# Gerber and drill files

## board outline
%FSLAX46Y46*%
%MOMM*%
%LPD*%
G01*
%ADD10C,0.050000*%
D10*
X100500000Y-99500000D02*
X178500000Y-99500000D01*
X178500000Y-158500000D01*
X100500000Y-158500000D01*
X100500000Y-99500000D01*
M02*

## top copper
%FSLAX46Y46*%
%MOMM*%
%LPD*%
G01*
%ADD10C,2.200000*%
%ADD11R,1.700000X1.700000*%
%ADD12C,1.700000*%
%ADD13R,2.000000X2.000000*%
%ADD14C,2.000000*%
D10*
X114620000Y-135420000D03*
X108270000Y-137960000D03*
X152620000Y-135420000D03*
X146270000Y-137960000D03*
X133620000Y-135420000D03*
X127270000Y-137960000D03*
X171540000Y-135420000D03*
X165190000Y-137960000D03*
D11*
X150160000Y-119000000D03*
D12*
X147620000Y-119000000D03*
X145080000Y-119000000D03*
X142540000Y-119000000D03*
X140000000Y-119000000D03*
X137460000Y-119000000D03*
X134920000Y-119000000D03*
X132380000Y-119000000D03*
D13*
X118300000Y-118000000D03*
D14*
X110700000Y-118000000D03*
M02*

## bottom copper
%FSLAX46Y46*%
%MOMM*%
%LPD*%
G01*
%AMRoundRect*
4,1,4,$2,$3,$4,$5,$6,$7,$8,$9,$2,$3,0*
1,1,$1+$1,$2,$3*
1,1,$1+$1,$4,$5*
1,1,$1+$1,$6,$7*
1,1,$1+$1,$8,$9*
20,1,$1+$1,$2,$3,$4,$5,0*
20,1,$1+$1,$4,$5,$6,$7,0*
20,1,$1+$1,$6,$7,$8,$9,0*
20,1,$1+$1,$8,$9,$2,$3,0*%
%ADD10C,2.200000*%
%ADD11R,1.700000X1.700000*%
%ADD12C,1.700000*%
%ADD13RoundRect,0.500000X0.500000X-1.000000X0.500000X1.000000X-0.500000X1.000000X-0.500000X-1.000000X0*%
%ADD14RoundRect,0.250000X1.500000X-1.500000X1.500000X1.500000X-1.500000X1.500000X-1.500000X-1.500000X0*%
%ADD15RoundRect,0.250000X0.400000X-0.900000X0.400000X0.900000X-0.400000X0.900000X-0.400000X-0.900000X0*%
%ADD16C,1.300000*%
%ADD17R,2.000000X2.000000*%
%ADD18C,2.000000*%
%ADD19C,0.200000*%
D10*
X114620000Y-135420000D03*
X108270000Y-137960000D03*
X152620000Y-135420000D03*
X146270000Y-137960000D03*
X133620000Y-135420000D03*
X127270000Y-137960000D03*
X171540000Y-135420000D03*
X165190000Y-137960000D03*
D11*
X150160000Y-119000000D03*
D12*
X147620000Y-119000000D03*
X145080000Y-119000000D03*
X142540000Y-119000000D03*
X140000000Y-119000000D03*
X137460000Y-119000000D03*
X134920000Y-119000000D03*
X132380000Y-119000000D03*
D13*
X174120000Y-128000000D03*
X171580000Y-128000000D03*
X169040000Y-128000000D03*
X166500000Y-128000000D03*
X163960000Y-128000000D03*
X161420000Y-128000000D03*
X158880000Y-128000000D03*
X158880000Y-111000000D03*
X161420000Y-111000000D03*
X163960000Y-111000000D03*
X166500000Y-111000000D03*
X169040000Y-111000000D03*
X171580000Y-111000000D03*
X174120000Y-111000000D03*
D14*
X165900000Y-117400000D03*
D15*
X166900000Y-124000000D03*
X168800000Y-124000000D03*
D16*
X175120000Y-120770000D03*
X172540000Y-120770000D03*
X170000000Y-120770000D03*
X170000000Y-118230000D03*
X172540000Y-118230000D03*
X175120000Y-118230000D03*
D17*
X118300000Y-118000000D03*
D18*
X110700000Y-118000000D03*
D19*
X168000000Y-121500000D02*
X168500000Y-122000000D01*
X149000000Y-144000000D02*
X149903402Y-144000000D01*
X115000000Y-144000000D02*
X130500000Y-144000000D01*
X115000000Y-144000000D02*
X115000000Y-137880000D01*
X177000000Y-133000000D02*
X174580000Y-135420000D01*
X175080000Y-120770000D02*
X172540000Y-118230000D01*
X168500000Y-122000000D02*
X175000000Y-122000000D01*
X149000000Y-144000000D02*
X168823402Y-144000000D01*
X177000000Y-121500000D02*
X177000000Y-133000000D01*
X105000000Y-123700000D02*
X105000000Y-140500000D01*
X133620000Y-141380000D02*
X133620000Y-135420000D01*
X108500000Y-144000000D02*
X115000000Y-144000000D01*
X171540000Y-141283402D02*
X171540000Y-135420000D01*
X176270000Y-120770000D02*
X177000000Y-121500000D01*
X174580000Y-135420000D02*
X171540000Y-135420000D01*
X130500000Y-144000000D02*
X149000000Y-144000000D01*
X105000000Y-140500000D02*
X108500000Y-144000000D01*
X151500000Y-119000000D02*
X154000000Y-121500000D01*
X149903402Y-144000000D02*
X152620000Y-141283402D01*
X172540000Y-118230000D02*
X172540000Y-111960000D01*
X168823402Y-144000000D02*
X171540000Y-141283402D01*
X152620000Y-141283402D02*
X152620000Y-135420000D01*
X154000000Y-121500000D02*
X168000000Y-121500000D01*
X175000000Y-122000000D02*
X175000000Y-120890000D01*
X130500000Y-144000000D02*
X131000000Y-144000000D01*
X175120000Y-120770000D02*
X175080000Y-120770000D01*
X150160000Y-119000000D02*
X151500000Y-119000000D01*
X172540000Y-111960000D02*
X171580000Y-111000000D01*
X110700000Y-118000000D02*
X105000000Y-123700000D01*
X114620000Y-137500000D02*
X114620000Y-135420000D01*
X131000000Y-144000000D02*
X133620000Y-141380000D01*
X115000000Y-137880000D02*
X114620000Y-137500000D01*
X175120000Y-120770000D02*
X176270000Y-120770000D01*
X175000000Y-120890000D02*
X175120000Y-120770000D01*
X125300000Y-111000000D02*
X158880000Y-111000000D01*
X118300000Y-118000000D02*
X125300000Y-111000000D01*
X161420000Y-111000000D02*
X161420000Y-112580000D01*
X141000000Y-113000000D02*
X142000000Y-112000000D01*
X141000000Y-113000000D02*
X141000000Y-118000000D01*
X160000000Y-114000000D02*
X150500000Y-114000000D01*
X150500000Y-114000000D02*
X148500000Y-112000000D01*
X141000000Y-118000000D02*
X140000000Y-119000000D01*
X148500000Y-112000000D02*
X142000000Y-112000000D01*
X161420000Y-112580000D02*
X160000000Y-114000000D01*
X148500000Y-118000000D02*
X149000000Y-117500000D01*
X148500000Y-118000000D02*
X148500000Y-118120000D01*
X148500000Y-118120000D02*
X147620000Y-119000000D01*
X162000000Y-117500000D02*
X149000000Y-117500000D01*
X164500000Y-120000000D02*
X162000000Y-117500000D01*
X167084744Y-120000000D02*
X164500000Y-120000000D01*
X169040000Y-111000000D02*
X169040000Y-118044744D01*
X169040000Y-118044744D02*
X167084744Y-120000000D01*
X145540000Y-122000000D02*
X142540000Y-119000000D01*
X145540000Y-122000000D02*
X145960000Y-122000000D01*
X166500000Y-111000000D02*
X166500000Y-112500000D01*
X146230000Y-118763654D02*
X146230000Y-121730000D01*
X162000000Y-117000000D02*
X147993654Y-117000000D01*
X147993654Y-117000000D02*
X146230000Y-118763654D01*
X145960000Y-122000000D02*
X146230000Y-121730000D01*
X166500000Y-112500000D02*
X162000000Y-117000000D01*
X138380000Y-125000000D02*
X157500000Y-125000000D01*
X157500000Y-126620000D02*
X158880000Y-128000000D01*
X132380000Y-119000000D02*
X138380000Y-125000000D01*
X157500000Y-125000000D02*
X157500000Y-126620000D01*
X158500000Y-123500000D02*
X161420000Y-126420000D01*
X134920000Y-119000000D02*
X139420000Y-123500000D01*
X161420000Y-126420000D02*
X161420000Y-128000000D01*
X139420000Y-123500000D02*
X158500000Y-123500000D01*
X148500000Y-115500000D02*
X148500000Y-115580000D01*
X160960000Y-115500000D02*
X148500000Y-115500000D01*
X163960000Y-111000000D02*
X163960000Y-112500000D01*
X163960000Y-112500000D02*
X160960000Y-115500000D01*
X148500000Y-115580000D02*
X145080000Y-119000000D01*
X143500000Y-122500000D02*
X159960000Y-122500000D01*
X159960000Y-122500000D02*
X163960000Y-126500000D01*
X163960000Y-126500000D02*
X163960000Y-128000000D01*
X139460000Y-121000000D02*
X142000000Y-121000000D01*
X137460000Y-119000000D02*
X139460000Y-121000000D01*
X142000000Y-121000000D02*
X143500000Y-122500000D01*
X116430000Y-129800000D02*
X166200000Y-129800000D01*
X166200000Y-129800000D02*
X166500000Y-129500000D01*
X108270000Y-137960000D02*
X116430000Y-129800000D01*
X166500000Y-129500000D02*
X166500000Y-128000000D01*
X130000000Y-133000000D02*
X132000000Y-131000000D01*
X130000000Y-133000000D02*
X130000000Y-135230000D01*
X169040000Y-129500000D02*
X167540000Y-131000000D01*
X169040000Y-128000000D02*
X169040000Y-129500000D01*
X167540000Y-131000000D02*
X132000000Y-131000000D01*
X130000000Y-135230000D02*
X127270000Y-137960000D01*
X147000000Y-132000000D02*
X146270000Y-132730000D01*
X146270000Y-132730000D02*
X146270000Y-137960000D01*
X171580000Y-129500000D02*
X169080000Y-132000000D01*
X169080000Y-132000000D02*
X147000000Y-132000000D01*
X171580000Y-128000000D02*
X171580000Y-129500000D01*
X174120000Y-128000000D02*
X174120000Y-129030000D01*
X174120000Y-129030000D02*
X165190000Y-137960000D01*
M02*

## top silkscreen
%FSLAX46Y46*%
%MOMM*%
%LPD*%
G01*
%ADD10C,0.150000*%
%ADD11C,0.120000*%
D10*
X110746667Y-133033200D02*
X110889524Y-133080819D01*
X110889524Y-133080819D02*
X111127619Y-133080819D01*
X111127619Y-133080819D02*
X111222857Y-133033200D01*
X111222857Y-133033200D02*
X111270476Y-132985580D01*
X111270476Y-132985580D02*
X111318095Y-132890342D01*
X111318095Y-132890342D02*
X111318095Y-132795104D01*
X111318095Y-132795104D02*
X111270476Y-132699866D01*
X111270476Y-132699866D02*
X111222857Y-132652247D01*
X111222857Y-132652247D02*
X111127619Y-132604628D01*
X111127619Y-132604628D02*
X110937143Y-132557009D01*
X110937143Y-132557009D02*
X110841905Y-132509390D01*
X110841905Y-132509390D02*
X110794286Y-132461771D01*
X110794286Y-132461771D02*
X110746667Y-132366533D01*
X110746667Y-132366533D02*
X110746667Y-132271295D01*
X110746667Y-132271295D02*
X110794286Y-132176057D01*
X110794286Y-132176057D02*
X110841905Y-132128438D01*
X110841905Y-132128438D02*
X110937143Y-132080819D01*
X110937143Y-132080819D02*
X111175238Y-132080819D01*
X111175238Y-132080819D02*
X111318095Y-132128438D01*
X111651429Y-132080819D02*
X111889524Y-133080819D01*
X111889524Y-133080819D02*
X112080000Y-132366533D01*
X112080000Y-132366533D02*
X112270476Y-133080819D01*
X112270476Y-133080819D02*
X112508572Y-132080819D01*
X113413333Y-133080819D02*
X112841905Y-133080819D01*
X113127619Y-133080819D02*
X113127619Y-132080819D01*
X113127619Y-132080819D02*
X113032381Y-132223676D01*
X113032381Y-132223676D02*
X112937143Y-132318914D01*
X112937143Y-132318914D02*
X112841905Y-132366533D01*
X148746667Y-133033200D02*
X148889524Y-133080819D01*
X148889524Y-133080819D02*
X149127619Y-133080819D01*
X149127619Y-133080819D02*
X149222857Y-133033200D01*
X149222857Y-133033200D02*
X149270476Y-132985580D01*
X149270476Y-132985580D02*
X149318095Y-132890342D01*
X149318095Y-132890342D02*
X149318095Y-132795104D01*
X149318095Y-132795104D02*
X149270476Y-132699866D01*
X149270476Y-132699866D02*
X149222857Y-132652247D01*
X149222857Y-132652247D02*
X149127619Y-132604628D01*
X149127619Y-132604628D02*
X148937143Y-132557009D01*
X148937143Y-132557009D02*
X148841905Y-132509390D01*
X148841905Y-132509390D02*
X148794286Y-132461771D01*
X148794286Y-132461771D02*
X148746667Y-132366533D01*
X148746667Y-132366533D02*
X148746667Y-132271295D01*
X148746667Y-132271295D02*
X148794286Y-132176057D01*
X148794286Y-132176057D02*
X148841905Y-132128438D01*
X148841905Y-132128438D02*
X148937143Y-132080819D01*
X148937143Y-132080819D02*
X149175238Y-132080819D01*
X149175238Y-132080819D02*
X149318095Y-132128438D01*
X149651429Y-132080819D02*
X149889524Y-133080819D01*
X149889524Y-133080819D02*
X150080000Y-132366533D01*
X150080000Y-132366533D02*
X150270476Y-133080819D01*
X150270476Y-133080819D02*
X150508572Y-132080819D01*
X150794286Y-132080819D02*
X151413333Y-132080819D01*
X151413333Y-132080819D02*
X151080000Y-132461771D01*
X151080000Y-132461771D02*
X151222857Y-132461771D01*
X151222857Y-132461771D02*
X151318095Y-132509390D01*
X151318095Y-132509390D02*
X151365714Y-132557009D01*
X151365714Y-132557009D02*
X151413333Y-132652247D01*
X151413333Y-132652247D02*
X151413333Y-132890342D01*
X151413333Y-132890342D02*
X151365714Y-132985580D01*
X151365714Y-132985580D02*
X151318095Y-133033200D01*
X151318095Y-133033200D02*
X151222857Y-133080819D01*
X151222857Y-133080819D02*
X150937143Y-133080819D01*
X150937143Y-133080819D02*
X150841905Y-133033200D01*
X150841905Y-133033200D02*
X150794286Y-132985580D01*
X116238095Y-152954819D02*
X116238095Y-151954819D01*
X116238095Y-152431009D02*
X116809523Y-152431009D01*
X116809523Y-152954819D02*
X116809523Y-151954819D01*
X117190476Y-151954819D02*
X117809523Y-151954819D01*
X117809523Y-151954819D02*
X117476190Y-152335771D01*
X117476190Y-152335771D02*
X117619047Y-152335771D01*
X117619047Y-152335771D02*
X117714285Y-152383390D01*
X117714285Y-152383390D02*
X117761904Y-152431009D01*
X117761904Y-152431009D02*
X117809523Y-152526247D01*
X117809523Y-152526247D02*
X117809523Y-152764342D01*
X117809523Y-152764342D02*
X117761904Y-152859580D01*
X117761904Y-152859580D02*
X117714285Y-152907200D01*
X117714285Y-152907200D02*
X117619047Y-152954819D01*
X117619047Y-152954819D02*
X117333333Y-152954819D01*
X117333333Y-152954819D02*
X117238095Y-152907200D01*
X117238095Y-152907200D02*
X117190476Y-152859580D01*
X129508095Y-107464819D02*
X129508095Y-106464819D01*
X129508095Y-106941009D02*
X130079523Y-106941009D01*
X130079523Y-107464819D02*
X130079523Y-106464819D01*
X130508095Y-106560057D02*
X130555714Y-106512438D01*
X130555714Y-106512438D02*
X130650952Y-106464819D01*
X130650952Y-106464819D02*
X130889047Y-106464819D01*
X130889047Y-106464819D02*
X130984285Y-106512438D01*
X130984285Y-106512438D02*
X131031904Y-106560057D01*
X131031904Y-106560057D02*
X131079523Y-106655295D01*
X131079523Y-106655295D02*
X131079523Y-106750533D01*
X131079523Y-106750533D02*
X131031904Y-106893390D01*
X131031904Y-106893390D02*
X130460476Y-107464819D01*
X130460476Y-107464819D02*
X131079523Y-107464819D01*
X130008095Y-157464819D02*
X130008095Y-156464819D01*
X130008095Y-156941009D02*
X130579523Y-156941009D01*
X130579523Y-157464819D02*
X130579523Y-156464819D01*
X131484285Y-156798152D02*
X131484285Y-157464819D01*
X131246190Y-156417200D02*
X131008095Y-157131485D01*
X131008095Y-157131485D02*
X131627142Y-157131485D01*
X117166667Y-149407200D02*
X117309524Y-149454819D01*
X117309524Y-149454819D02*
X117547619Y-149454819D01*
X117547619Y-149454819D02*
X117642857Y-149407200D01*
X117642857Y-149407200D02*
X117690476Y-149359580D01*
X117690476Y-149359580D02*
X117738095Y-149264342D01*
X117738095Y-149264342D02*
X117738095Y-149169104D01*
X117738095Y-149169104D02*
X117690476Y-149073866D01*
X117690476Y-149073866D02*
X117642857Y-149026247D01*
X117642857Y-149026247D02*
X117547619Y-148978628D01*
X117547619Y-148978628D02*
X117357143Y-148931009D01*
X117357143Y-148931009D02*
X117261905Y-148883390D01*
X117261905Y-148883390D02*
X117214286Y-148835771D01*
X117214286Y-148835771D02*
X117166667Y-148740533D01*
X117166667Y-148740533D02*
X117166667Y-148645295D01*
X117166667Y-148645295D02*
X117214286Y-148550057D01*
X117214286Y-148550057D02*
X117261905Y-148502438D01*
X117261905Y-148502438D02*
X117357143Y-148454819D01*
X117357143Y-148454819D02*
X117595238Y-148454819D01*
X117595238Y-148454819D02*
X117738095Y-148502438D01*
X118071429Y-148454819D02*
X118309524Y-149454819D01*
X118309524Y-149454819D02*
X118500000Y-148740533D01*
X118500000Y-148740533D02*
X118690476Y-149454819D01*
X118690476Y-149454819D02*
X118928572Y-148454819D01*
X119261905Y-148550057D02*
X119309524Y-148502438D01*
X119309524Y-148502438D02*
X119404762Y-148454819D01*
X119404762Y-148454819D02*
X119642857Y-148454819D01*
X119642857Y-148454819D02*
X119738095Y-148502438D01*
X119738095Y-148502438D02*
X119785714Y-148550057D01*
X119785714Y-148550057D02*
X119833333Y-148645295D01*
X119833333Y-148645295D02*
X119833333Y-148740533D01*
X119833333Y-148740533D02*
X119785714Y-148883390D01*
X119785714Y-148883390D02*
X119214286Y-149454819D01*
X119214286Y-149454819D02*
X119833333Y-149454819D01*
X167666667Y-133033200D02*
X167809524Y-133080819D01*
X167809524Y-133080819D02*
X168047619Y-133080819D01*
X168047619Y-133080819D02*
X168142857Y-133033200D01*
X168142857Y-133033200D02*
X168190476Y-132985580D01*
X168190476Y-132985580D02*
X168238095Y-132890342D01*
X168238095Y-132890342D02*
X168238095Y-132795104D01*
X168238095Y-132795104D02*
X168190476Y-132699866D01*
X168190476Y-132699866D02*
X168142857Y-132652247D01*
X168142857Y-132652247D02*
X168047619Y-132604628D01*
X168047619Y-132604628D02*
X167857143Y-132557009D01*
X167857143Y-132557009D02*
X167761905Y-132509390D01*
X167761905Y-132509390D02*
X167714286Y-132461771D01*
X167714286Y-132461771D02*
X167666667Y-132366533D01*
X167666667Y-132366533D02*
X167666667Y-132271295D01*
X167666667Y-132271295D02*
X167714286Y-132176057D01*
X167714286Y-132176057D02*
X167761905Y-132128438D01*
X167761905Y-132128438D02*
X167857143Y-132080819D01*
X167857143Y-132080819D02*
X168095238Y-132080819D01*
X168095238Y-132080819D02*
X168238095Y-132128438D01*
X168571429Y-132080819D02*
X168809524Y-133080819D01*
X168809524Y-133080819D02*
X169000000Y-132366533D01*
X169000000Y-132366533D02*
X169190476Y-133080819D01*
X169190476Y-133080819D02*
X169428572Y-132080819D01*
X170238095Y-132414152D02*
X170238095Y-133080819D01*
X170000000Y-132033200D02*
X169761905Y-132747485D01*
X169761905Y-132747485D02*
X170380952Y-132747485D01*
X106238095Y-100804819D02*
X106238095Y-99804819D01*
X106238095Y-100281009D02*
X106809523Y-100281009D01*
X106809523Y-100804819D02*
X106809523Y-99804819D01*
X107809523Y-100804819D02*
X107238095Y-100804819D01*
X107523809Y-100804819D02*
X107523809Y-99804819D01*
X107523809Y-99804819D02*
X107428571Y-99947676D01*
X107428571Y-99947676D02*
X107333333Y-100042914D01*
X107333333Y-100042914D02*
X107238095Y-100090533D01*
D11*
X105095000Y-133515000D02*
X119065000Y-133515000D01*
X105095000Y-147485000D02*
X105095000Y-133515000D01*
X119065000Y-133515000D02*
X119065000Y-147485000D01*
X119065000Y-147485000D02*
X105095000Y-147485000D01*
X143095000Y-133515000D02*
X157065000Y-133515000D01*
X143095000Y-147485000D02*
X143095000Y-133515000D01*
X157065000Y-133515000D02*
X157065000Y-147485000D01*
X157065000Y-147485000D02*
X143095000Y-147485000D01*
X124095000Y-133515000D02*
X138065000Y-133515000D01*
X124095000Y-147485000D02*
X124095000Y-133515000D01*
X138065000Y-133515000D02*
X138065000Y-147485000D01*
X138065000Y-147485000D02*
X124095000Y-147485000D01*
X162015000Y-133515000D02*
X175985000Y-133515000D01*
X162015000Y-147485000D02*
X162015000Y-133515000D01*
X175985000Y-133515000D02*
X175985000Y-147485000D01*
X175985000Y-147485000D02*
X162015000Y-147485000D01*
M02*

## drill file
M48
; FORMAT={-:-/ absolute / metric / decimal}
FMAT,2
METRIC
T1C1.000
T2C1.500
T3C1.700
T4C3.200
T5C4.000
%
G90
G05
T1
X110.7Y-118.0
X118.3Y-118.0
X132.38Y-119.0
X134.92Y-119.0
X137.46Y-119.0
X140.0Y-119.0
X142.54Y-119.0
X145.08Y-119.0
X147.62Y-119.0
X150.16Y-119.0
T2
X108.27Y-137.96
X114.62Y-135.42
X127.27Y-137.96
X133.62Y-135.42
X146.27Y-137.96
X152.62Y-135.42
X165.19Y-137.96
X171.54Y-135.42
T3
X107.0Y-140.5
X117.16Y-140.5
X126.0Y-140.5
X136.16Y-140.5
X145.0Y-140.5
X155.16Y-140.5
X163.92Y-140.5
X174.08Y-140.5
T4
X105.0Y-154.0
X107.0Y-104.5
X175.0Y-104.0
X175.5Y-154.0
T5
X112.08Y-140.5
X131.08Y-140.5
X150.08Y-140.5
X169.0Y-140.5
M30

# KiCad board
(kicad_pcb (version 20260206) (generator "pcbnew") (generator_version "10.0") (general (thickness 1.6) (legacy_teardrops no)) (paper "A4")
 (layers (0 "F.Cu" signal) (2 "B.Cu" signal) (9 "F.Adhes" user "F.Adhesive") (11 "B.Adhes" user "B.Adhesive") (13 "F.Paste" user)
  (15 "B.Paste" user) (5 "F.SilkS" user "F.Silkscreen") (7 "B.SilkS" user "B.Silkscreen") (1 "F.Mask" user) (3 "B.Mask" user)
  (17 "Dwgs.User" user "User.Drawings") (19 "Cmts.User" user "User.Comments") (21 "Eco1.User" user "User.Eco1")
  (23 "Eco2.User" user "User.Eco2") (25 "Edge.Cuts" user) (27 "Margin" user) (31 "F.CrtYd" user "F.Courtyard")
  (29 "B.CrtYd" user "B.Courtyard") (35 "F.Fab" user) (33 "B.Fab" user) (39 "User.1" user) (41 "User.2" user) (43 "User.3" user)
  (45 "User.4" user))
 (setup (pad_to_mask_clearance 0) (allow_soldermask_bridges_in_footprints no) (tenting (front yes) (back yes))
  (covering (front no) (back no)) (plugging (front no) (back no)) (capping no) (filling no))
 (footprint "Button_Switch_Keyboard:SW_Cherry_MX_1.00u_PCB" (layer "F.Cu") (at 114.62 135.42)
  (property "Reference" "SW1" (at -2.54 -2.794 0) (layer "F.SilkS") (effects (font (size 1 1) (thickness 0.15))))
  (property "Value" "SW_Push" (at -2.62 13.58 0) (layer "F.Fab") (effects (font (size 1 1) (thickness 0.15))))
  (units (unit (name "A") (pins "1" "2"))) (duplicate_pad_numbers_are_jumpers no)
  (fp_line (start -9.525 -1.905) (end 4.445 -1.905) (stroke (width 0.12) (type solid)) (layer "F.SilkS"))
  (fp_line (start -9.525 12.065) (end -9.525 -1.905) (stroke (width 0.12) (type solid)) (layer "F.SilkS"))
  (fp_line (start 4.445 -1.905) (end 4.445 12.065) (stroke (width 0.12) (type solid)) (layer "F.SilkS"))
  (fp_line (start 4.445 12.065) (end -9.525 12.065) (stroke (width 0.12) (type solid)) (layer "F.SilkS"))
  (pad "" np_thru_hole circle (at -7.62 5.08) (size 1.7 1.7) (drill 1.7) (layers "*.Cu" "*.Mask"))
  (pad "" np_thru_hole circle (at -2.54 5.08) (size 4 4) (drill 4) (layers "*.Cu" "*.Mask"))
  (pad "" np_thru_hole circle (at 2.54 5.08) (size 1.7 1.7) (drill 1.7) (layers "*.Cu" "*.Mask"))
  (pad "1" thru_hole circle (at 0 0) (size 2.2 2.2) (drill 1.5) (layers "*.Cu" "*.Mask") (remove_unused_layers no) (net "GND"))
  (pad "2" thru_hole circle (at -6.35 2.54) (size 2.2 2.2) (drill 1.5) (layers "*.Cu" "*.Mask") (remove_unused_layers no)
   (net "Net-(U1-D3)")))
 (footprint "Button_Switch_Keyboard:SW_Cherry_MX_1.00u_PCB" (layer "F.Cu") (at 152.62 135.42)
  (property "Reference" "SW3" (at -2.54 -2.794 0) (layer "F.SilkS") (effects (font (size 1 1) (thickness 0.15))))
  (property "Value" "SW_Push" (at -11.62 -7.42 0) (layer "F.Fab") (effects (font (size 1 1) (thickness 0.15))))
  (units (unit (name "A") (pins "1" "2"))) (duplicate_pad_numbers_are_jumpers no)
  (fp_line (start -9.525 -1.905) (end 4.445 -1.905) (stroke (width 0.12) (type solid)) (layer "F.SilkS"))
  (fp_line (start -9.525 12.065) (end -9.525 -1.905) (stroke (width 0.12) (type solid)) (layer "F.SilkS"))
  (fp_line (start 4.445 -1.905) (end 4.445 12.065) (stroke (width 0.12) (type solid)) (layer "F.SilkS"))
  (fp_line (start 4.445 12.065) (end -9.525 12.065) (stroke (width 0.12) (type solid)) (layer "F.SilkS"))
  (pad "" np_thru_hole circle (at -7.62 5.08) (size 1.7 1.7) (drill 1.7) (layers "*.Cu" "*.Mask"))
  (pad "" np_thru_hole circle (at -2.54 5.08) (size 4 4) (drill 4) (layers "*.Cu" "*.Mask"))
  (pad "" np_thru_hole circle (at 2.54 5.08) (size 1.7 1.7) (drill 1.7) (layers "*.Cu" "*.Mask"))
  (pad "1" thru_hole circle (at 0 0) (size 2.2 2.2) (drill 1.5) (layers "*.Cu" "*.Mask") (remove_unused_layers no) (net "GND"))
  (pad "2" thru_hole circle (at -6.35 2.54) (size 2.2 2.2) (drill 1.5) (layers "*.Cu" "*.Mask") (remove_unused_layers no)
   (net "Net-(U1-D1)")))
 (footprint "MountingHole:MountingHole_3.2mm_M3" (layer "F.Cu") (at 105 154)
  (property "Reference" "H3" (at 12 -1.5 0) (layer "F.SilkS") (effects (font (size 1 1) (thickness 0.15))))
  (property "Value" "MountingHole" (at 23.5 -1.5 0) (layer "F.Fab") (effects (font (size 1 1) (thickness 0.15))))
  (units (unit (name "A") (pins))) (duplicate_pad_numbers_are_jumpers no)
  (pad "" np_thru_hole circle (at 0 0) (size 3.2 3.2) (drill 3.2) (layers "*.Cu" "*.Mask")))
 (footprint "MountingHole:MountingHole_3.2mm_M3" (layer "F.Cu") (at 175 104)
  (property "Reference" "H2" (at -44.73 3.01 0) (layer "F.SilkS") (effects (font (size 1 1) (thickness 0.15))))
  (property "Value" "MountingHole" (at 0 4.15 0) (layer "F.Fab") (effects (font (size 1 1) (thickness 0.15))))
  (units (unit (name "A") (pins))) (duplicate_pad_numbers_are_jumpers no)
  (pad "" np_thru_hole circle (at 0 0) (size 3.2 3.2) (drill 3.2) (layers "*.Cu" "*.Mask")))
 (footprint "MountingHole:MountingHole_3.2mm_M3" (layer "F.Cu") (at 175.5 154)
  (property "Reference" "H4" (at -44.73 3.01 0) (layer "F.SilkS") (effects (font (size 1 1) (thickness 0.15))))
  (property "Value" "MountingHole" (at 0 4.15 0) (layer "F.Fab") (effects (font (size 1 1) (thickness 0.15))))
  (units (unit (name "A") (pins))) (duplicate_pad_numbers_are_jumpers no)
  (pad "" np_thru_hole circle (at 0 0) (size 3.2 3.2) (drill 3.2) (layers "*.Cu" "*.Mask")))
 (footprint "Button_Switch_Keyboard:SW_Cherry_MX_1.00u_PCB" (layer "F.Cu") (at 133.62 135.42)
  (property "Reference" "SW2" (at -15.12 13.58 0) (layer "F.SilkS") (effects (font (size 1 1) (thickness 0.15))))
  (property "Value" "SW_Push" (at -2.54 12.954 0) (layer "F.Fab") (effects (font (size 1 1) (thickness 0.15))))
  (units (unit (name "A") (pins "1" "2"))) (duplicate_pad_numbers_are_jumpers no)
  (fp_line (start -9.525 -1.905) (end 4.445 -1.905) (stroke (width 0.12) (type solid)) (layer "F.SilkS"))
  (fp_line (start -9.525 12.065) (end -9.525 -1.905) (stroke (width 0.12) (type solid)) (layer "F.SilkS"))
  (fp_line (start 4.445 -1.905) (end 4.445 12.065) (stroke (width 0.12) (type solid)) (layer "F.SilkS"))
  (fp_line (start 4.445 12.065) (end -9.525 12.065) (stroke (width 0.12) (type solid)) (layer "F.SilkS"))
  (pad "" np_thru_hole circle (at -7.62 5.08) (size 1.7 1.7) (drill 1.7) (layers "*.Cu" "*.Mask"))
  (pad "" np_thru_hole circle (at -2.54 5.08) (size 4 4) (drill 4) (layers "*.Cu" "*.Mask"))
  (pad "" np_thru_hole circle (at 2.54 5.08) (size 1.7 1.7) (drill 1.7) (layers "*.Cu" "*.Mask"))
  (pad "1" thru_hole circle (at 0 0) (size 2.2 2.2) (drill 1.5) (layers "*.Cu" "*.Mask") (remove_unused_layers no) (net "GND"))
  (pad "2" thru_hole circle (at -6.35 2.54) (size 2.2 2.2) (drill 1.5) (layers "*.Cu" "*.Mask") (remove_unused_layers no)
   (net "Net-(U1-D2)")))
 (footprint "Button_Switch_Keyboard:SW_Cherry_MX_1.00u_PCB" (layer "F.Cu") (at 171.54 135.42)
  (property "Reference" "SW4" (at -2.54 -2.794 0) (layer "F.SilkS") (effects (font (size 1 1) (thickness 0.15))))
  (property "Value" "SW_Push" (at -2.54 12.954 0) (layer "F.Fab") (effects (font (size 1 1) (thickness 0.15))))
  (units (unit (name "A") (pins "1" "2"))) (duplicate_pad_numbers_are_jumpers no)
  (fp_line (start -9.525 -1.905) (end 4.445 -1.905) (stroke (width 0.12) (type solid)) (layer "F.SilkS"))
  (fp_line (start -9.525 12.065) (end -9.525 -1.905) (stroke (width 0.12) (type solid)) (layer "F.SilkS"))
  (fp_line (start 4.445 -1.905) (end 4.445 12.065) (stroke (width 0.12) (type solid)) (layer "F.SilkS"))
  (fp_line (start 4.445 12.065) (end -9.525 12.065) (stroke (width 0.12) (type solid)) (layer "F.SilkS"))
  (pad "" np_thru_hole circle (at -7.62 5.08) (size 1.7 1.7) (drill 1.7) (layers "*.Cu" "*.Mask"))
  (pad "" np_thru_hole circle (at -2.54 5.08) (size 4 4) (drill 4) (layers "*.Cu" "*.Mask"))
  (pad "" np_thru_hole circle (at 2.54 5.08) (size 1.7 1.7) (drill 1.7) (layers "*.Cu" "*.Mask"))
  (pad "1" thru_hole circle (at 0 0) (size 2.2 2.2) (drill 1.5) (layers "*.Cu" "*.Mask") (remove_unused_layers no) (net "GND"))
  (pad "2" thru_hole circle (at -6.35 2.54) (size 2.2 2.2) (drill 1.5) (layers "*.Cu" "*.Mask") (remove_unused_layers no)
   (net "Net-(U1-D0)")))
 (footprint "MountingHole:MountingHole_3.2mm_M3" (layer "F.Cu") (at 107 104.5)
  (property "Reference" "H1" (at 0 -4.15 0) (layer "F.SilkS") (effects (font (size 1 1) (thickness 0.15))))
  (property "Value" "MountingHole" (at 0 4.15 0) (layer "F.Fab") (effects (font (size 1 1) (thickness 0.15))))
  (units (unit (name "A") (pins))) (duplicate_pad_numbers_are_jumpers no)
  (pad "" np_thru_hole circle (at 0 0) (size 3.2 3.2) (drill 3.2) (layers "*.Cu" "*.Mask")))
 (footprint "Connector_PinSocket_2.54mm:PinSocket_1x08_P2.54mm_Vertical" (layer "B.Cu") (at 150.16 119 90)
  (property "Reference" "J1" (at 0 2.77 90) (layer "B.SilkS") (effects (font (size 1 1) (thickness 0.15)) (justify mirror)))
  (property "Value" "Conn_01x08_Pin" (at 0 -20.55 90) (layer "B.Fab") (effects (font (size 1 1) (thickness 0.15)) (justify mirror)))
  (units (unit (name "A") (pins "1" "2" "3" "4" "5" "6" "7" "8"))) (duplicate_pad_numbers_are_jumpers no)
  (pad "1" thru_hole rect (at 0 0 90) (size 1.7 1.7) (drill 1) (layers "*.Cu" "*.Mask") (remove_unused_layers no) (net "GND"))
  (pad "2" thru_hole circle (at 0 -2.54 90) (size 1.7 1.7) (drill 1) (layers "*.Cu" "*.Mask") (remove_unused_layers no) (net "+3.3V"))
  (pad "3" thru_hole circle (at 0 -5.08 90) (size 1.7 1.7) (drill 1) (layers "*.Cu" "*.Mask") (remove_unused_layers no) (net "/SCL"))
  (pad "4" thru_hole circle (at 0 -7.62 90) (size 1.7 1.7) (drill 1) (layers "*.Cu" "*.Mask") (remove_unused_layers no) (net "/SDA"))
  (pad "5" thru_hole circle (at 0 -10.16 90) (size 1.7 1.7) (drill 1) (layers "*.Cu" "*.Mask") (remove_unused_layers no) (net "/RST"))
  (pad "6" thru_hole circle (at 0 -12.7 90) (size 1.7 1.7) (drill 1) (layers "*.Cu" "*.Mask") (remove_unused_layers no) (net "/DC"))
  (pad "7" thru_hole circle (at 0 -15.24 90) (size 1.7 1.7) (drill 1) (layers "*.Cu" "*.Mask") (remove_unused_layers no) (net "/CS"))
  (pad "8" thru_hole circle (at 0 -17.78 90) (size 1.7 1.7) (drill 1) (layers "*.Cu" "*.Mask") (remove_unused_layers no) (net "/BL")))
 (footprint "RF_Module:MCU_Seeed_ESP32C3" (layer "B.Cu") (at 166.5 119.5 90)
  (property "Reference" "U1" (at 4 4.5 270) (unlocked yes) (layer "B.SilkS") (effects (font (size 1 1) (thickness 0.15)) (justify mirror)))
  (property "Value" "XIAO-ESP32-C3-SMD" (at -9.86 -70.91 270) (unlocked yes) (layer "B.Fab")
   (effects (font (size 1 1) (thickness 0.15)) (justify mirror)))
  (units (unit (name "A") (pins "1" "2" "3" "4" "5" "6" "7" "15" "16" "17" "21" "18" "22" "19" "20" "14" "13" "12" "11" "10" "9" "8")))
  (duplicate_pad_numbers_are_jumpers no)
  (pad "" smd roundrect (at 1.1 -1.6 90) (size 1.5 1.5) (layers "B.Paste") (roundrect_rratio 0.1666666667))
  (pad "" smd roundrect (at 1.1 0.4 90) (size 1.5 1.5) (layers "B.Paste") (roundrect_rratio 0.1666666667))
  (pad "" smd roundrect (at 3.1 -1.6 90) (size 1.5 1.5) (layers "B.Paste") (roundrect_rratio 0.1666666667))
  (pad "" smd roundrect (at 3.1 0.4 90) (size 1.5 1.5) (layers "B.Paste") (roundrect_rratio 0.1666666667))
  (pad "1" smd roundrect (at -8.5 7.62 90) (size 3 2) (layers "B.Cu" "B.Mask" "B.Paste") (roundrect_rratio 0.25) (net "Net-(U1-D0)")
   (thermal_bridge_angle 45))
  (pad "2" smd roundrect (at -8.5 5.08 90) (size 3 2) (layers "B.Cu" "B.Mask" "B.Paste") (roundrect_rratio 0.25) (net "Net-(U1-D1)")
   (thermal_bridge_angle 45))
  (pad "3" smd roundrect (at -8.5 2.54 90) (size 3 2) (layers "B.Cu" "B.Mask" "B.Paste") (roundrect_rratio 0.25) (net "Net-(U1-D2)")
   (thermal_bridge_angle 45))
  (pad "4" smd roundrect (at -8.5 0 90) (size 3 2) (layers "B.Cu" "B.Mask" "B.Paste") (roundrect_rratio 0.25) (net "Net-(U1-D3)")
   (thermal_bridge_angle 45))
  (pad "5" smd roundrect (at -8.5 -2.54 90) (size 3 2) (layers "B.Cu" "B.Mask" "B.Paste") (roundrect_rratio 0.25) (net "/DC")
   (thermal_bridge_angle 45))
  (pad "6" smd roundrect (at -8.5 -5.08 90) (size 3 2) (layers "B.Cu" "B.Mask" "B.Paste") (roundrect_rratio 0.25) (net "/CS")
   (thermal_bridge_angle 45))
  (pad "7" smd roundrect (at -8.5 -7.62 90) (size 3 2) (layers "B.Cu" "B.Mask" "B.Paste") (roundrect_rratio 0.25) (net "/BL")
   (thermal_bridge_angle 45))
  (pad "8" smd roundrect (at 8.5 -7.62 90) (size 3 2) (layers "B.Cu" "B.Mask" "B.Paste") (roundrect_rratio 0.25) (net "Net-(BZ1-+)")
   (thermal_bridge_angle 45))
  (pad "9" smd roundrect (at 8.5 -5.08 90) (size 3 2) (layers "B.Cu" "B.Mask" "B.Paste") (roundrect_rratio 0.25) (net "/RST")
   (thermal_bridge_angle 45))
  (pad "10" smd roundrect (at 8.5 -2.54 90) (size 3 2) (layers "B.Cu" "B.Mask" "B.Paste") (roundrect_rratio 0.25) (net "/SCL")
   (thermal_bridge_angle 45))
  (pad "11" smd roundrect (at 8.5 0 90) (size 3 2) (layers "B.Cu" "B.Mask" "B.Paste") (roundrect_rratio 0.25) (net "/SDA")
   (thermal_bridge_angle 45))
  (pad "12" smd roundrect (at 8.5 2.54 90) (size 3 2) (layers "B.Cu" "B.Mask" "B.Paste") (roundrect_rratio 0.25) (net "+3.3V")
   (thermal_bridge_angle 45))
  (pad "13" smd roundrect (at 8.5 5.08 90) (size 3 2) (layers "B.Cu" "B.Mask" "B.Paste") (roundrect_rratio 0.25) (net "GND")
   (thermal_bridge_angle 45))
  (pad "14" smd roundrect (at 8.5 7.62 90) (size 3 2) (layers "B.Cu" "B.Mask" "B.Paste") (roundrect_rratio 0.25)
   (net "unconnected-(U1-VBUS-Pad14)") (thermal_bridge_angle 45))
  (pad "15" smd roundrect (at 2.1 -0.6 90) (size 3.5 3.5) (layers "B.Cu" "B.Mask") (roundrect_rratio 0.07142857143)
   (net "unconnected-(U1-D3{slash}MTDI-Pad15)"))
  (pad "16" smd roundrect (at -4.5 0.4 90) (size 2.3 1.3) (layers "B.Cu" "B.Mask" "B.Paste") (roundrect_rratio 0.1923076923)
   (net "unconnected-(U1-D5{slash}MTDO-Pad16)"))
  (pad "17" smd roundrect (at -4.5 2.3 90) (size 2.3 1.3) (layers "B.Cu" "B.Mask" "B.Paste") (roundrect_rratio 0.1923076923)
   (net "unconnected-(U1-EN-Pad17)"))
  (pad "18" smd circle (at -1.27 8.62 90) (size 1.3 1.3) (layers "B.Cu" "B.Mask" "B.Paste") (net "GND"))
  (pad "19" smd circle (at -1.27 6.04 90) (size 1.3 1.3) (layers "B.Cu" "B.Mask" "B.Paste") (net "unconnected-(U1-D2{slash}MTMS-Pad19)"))
  (pad "20" smd circle (at -1.27 3.5 90) (size 1.3 1.3) (layers "B.Cu" "B.Mask" "B.Paste") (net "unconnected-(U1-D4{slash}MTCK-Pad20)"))
  (pad "21" smd circle (at 1.27 3.5 90) (size 1.3 1.3) (layers "B.Cu" "B.Mask" "B.Paste") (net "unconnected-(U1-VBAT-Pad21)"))
  (pad "22" smd circle (at 1.27 6.04 90) (size 1.3 1.3) (layers "B.Cu" "B.Mask" "B.Paste") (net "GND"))
  (pad "23" smd circle (at 1.27 8.62 90) (size 1.3 1.3) (layers "B.Cu" "B.Mask" "B.Paste")))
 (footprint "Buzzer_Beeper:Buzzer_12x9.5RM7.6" (layer "B.Cu") (at 118.3 118 180)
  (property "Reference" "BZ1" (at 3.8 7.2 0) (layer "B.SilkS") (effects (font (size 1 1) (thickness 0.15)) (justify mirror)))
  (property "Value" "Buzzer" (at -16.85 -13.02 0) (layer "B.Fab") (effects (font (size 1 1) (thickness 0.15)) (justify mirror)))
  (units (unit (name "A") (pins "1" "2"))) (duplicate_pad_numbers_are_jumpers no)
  (pad "1" thru_hole rect (at 0 0 180) (size 2 2) (drill 1) (layers "*.Cu" "*.Mask") (remove_unused_layers no) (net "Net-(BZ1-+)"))
  (pad "2" thru_hole circle (at 7.6 0 180) (size 2 2) (drill 1) (layers "*.Cu" "*.Mask") (remove_unused_layers no) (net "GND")))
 (gr_rect (start 100.5 99.5) (end 178.5 158.5) (stroke (width 0.05) (type default)) (fill no) (layer "Edge.Cuts"))
 (segment (start 168 121.5) (end 168.5 122) (width 0.2) (layer "B.Cu") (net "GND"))
 (segment (start 149 144) (end 149.903402 144) (width 0.2) (layer "B.Cu") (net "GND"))
 (segment (start 115 144) (end 130.5 144) (width 0.2) (layer "B.Cu") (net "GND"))
 (segment (start 115 144) (end 115 137.88) (width 0.2) (layer "B.Cu") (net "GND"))
 (segment (start 177 133) (end 174.58 135.42) (width 0.2) (layer "B.Cu") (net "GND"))
 (segment (start 175.08 120.77) (end 172.54 118.23) (width 0.2) (layer "B.Cu") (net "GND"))
 (segment (start 168.5 122) (end 175 122) (width 0.2) (layer "B.Cu") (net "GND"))
 (segment (start 149 144) (end 168.823402 144) (width 0.2) (layer "B.Cu") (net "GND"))
 (segment (start 177 121.5) (end 177 133) (width 0.2) (layer "B.Cu") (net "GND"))
 (segment (start 105 123.7) (end 105 140.5) (width 0.2) (layer "B.Cu") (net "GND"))
 (segment (start 133.62 141.38) (end 133.62 135.42) (width 0.2) (layer "B.Cu") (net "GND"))
 (segment (start 108.5 144) (end 115 144) (width 0.2) (layer "B.Cu") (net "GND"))
 (segment (start 171.54 141.283402) (end 171.54 135.42) (width 0.2) (layer "B.Cu") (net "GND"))
 (segment (start 176.27 120.77) (end 177 121.5) (width 0.2) (layer "B.Cu") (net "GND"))
 (segment (start 174.58 135.42) (end 171.54 135.42) (width 0.2) (layer "B.Cu") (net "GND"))
 (segment (start 130.5 144) (end 149 144) (width 0.2) (layer "B.Cu") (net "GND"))
 (segment (start 105 140.5) (end 108.5 144) (width 0.2) (layer "B.Cu") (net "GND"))
 (segment (start 151.5 119) (end 154 121.5) (width 0.2) (layer "B.Cu") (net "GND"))
 (segment (start 149.903402 144) (end 152.62 141.283402) (width 0.2) (layer "B.Cu") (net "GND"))
 (segment (start 172.54 118.23) (end 172.54 111.96) (width 0.2) (layer "B.Cu") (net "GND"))
 (segment (start 168.823402 144) (end 171.54 141.283402) (width 0.2) (layer "B.Cu") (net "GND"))
 (segment (start 152.62 141.283402) (end 152.62 135.42) (width 0.2) (layer "B.Cu") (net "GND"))
 (segment (start 154 121.5) (end 168 121.5) (width 0.2) (layer "B.Cu") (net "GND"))
 (segment (start 175 122) (end 175 120.89) (width 0.2) (layer "B.Cu") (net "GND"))
 (segment (start 130.5 144) (end 131 144) (width 0.2) (layer "B.Cu") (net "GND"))
 (segment (start 175.12 120.77) (end 175.08 120.77) (width 0.2) (layer "B.Cu") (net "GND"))
 (segment (start 150.16 119) (end 151.5 119) (width 0.2) (layer "B.Cu") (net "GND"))
 (segment (start 172.54 111.96) (end 171.58 111) (width 0.2) (layer "B.Cu") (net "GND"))
 (segment (start 110.7 118) (end 105 123.7) (width 0.2) (layer "B.Cu") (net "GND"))
 (segment (start 114.62 137.5) (end 114.62 135.42) (width 0.2) (layer "B.Cu") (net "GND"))
 (segment (start 131 144) (end 133.62 141.38) (width 0.2) (layer "B.Cu") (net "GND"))
 (segment (start 115 137.88) (end 114.62 137.5) (width 0.2) (layer "B.Cu") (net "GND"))
 (segment (start 175.12 120.77) (end 176.27 120.77) (width 0.2) (layer "B.Cu") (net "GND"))
 (segment (start 175 120.89) (end 175.12 120.77) (width 0.2) (layer "B.Cu") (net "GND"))
 (segment (start 125.3 111) (end 158.88 111) (width 0.2) (layer "B.Cu") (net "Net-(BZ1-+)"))
 (segment (start 118.3 118) (end 125.3 111) (width 0.2) (layer "B.Cu") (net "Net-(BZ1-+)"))
 (segment (start 161.42 111) (end 161.42 112.58) (width 0.2) (layer "B.Cu") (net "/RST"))
 (segment (start 141 113) (end 142 112) (width 0.2) (layer "B.Cu") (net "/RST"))
 (segment (start 141 113) (end 141 118) (width 0.2) (layer "B.Cu") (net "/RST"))
 (segment (start 160 114) (end 150.5 114) (width 0.2) (layer "B.Cu") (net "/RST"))
 (segment (start 150.5 114) (end 148.5 112) (width 0.2) (layer "B.Cu") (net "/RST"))
 (segment (start 141 118) (end 140 119) (width 0.2) (layer "B.Cu") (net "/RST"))
 (segment (start 148.5 112) (end 142 112) (width 0.2) (layer "B.Cu") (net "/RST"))
 (segment (start 161.42 112.58) (end 160 114) (width 0.2) (layer "B.Cu") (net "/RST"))
 (segment (start 148.5 118) (end 149 117.5) (width 0.2) (layer "B.Cu") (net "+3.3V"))
 (segment (start 148.5 118) (end 148.5 118.12) (width 0.2) (layer "B.Cu") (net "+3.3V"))
 (segment (start 148.5 118.12) (end 147.62 119) (width 0.2) (layer "B.Cu") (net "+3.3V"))
 (segment (start 162 117.5) (end 149 117.5) (width 0.2) (layer "B.Cu") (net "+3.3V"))
 (segment (start 164.5 120) (end 162 117.5) (width 0.2) (layer "B.Cu") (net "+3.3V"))
 (segment (start 167.084744 120) (end 164.5 120) (width 0.2) (layer "B.Cu") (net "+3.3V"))
 (segment (start 169.04 111) (end 169.04 118.044744) (width 0.2) (layer "B.Cu") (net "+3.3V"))
 (segment (start 169.04 118.044744) (end 167.084744 120) (width 0.2) (layer "B.Cu") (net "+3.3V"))
 (segment (start 145.54 122) (end 142.54 119) (width 0.2) (layer "B.Cu") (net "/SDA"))
 (segment (start 145.54 122) (end 145.96 122) (width 0.2) (layer "B.Cu") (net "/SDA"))
 (segment (start 166.5 111) (end 166.5 112.5) (width 0.2) (layer "B.Cu") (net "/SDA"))
 (segment (start 146.23 118.763654) (end 146.23 121.73) (width 0.2) (layer "B.Cu") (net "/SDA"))
 (segment (start 162 117) (end 147.993654 117) (width 0.2) (layer "B.Cu") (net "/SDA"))
 (segment (start 147.993654 117) (end 146.23 118.763654) (width 0.2) (layer "B.Cu") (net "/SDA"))
 (segment (start 145.96 122) (end 146.23 121.73) (width 0.2) (layer "B.Cu") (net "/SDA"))
 (segment (start 166.5 112.5) (end 162 117) (width 0.2) (layer "B.Cu") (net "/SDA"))
 (segment (start 138.38 125) (end 157.5 125) (width 0.2) (layer "B.Cu") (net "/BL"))
 (segment (start 157.5 126.62) (end 158.88 128) (width 0.2) (layer "B.Cu") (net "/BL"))
 (segment (start 132.38 119) (end 138.38 125) (width 0.2) (layer "B.Cu") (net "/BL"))
 (segment (start 157.5 125) (end 157.5 126.62) (width 0.2) (layer "B.Cu") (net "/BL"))
 (segment (start 158.5 123.5) (end 161.42 126.42) (width 0.2) (layer "B.Cu") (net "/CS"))
 (segment (start 134.92 119) (end 139.42 123.5) (width 0.2) (layer "B.Cu") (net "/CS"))
 (segment (start 161.42 126.42) (end 161.42 128) (width 0.2) (layer "B.Cu") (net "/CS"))
 (segment (start 139.42 123.5) (end 158.5 123.5) (width 0.2) (layer "B.Cu") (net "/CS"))
 (segment (start 148.5 115.5) (end 148.5 115.58) (width 0.2) (layer "B.Cu") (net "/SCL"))
 (segment (start 160.96 115.5) (end 148.5 115.5) (width 0.2) (layer "B.Cu") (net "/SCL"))
 (segment (start 163.96 111) (end 163.96 112.5) (width 0.2) (layer "B.Cu") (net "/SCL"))
 (segment (start 163.96 112.5) (end 160.96 115.5) (width 0.2) (layer "B.Cu") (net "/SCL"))
 (segment (start 148.5 115.58) (end 145.08 119) (width 0.2) (layer "B.Cu") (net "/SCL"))
 (segment (start 143.5 122.5) (end 159.96 122.5) (width 0.2) (layer "B.Cu") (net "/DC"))
 (segment (start 159.96 122.5) (end 163.96 126.5) (width 0.2) (layer "B.Cu") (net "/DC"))
 (segment (start 163.96 126.5) (end 163.96 128) (width 0.2) (layer "B.Cu") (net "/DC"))
 (segment (start 139.46 121) (end 142 121) (width 0.2) (layer "B.Cu") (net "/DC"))
 (segment (start 137.46 119) (end 139.46 121) (width 0.2) (layer "B.Cu") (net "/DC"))
 (segment (start 142 121) (end 143.5 122.5) (width 0.2) (layer "B.Cu") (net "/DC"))
 (segment (start 116.43 129.8) (end 166.2 129.8) (width 0.2) (layer "B.Cu") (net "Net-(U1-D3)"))
 (segment (start 166.2 129.8) (end 166.5 129.5) (width 0.2) (layer "B.Cu") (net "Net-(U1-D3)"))
 (segment (start 108.27 137.96) (end 116.43 129.8) (width 0.2) (layer "B.Cu") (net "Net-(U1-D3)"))
 (segment (start 166.5 129.5) (end 166.5 128) (width 0.2) (layer "B.Cu") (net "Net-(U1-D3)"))
 (segment (start 130 133) (end 132 131) (width 0.2) (layer "B.Cu") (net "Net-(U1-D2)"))
 (segment (start 130 133) (end 130 135.23) (width 0.2) (layer "B.Cu") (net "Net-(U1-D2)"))
 (segment (start 169.04 129.5) (end 167.54 131) (width 0.2) (layer "B.Cu") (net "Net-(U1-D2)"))
 (segment (start 169.04 128) (end 169.04 129.5) (width 0.2) (layer "B.Cu") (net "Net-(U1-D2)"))
 (segment (start 167.54 131) (end 132 131) (width 0.2) (layer "B.Cu") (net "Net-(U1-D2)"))
 (segment (start 130 135.23) (end 127.27 137.96) (width 0.2) (layer "B.Cu") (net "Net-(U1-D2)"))
 (segment (start 147 132) (end 146.27 132.73) (width 0.2) (layer "B.Cu") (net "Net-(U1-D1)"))
 (segment (start 146.27 132.73) (end 146.27 137.96) (width 0.2) (layer "B.Cu") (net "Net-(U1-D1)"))
 (segment (start 171.58 129.5) (end 169.08 132) (width 0.2) (layer "B.Cu") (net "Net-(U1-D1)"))
 (segment (start 169.08 132) (end 147 132) (width 0.2) (layer "B.Cu") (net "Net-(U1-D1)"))
 (segment (start 171.58 128) (end 171.58 129.5) (width 0.2) (layer "B.Cu") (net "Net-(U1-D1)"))
 (segment (start 174.12 128) (end 174.12 129.03) (width 0.2) (layer "B.Cu") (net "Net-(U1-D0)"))
 (segment (start 174.12 129.03) (end 165.19 137.96) (width 0.2) (layer "B.Cu") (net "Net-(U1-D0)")))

